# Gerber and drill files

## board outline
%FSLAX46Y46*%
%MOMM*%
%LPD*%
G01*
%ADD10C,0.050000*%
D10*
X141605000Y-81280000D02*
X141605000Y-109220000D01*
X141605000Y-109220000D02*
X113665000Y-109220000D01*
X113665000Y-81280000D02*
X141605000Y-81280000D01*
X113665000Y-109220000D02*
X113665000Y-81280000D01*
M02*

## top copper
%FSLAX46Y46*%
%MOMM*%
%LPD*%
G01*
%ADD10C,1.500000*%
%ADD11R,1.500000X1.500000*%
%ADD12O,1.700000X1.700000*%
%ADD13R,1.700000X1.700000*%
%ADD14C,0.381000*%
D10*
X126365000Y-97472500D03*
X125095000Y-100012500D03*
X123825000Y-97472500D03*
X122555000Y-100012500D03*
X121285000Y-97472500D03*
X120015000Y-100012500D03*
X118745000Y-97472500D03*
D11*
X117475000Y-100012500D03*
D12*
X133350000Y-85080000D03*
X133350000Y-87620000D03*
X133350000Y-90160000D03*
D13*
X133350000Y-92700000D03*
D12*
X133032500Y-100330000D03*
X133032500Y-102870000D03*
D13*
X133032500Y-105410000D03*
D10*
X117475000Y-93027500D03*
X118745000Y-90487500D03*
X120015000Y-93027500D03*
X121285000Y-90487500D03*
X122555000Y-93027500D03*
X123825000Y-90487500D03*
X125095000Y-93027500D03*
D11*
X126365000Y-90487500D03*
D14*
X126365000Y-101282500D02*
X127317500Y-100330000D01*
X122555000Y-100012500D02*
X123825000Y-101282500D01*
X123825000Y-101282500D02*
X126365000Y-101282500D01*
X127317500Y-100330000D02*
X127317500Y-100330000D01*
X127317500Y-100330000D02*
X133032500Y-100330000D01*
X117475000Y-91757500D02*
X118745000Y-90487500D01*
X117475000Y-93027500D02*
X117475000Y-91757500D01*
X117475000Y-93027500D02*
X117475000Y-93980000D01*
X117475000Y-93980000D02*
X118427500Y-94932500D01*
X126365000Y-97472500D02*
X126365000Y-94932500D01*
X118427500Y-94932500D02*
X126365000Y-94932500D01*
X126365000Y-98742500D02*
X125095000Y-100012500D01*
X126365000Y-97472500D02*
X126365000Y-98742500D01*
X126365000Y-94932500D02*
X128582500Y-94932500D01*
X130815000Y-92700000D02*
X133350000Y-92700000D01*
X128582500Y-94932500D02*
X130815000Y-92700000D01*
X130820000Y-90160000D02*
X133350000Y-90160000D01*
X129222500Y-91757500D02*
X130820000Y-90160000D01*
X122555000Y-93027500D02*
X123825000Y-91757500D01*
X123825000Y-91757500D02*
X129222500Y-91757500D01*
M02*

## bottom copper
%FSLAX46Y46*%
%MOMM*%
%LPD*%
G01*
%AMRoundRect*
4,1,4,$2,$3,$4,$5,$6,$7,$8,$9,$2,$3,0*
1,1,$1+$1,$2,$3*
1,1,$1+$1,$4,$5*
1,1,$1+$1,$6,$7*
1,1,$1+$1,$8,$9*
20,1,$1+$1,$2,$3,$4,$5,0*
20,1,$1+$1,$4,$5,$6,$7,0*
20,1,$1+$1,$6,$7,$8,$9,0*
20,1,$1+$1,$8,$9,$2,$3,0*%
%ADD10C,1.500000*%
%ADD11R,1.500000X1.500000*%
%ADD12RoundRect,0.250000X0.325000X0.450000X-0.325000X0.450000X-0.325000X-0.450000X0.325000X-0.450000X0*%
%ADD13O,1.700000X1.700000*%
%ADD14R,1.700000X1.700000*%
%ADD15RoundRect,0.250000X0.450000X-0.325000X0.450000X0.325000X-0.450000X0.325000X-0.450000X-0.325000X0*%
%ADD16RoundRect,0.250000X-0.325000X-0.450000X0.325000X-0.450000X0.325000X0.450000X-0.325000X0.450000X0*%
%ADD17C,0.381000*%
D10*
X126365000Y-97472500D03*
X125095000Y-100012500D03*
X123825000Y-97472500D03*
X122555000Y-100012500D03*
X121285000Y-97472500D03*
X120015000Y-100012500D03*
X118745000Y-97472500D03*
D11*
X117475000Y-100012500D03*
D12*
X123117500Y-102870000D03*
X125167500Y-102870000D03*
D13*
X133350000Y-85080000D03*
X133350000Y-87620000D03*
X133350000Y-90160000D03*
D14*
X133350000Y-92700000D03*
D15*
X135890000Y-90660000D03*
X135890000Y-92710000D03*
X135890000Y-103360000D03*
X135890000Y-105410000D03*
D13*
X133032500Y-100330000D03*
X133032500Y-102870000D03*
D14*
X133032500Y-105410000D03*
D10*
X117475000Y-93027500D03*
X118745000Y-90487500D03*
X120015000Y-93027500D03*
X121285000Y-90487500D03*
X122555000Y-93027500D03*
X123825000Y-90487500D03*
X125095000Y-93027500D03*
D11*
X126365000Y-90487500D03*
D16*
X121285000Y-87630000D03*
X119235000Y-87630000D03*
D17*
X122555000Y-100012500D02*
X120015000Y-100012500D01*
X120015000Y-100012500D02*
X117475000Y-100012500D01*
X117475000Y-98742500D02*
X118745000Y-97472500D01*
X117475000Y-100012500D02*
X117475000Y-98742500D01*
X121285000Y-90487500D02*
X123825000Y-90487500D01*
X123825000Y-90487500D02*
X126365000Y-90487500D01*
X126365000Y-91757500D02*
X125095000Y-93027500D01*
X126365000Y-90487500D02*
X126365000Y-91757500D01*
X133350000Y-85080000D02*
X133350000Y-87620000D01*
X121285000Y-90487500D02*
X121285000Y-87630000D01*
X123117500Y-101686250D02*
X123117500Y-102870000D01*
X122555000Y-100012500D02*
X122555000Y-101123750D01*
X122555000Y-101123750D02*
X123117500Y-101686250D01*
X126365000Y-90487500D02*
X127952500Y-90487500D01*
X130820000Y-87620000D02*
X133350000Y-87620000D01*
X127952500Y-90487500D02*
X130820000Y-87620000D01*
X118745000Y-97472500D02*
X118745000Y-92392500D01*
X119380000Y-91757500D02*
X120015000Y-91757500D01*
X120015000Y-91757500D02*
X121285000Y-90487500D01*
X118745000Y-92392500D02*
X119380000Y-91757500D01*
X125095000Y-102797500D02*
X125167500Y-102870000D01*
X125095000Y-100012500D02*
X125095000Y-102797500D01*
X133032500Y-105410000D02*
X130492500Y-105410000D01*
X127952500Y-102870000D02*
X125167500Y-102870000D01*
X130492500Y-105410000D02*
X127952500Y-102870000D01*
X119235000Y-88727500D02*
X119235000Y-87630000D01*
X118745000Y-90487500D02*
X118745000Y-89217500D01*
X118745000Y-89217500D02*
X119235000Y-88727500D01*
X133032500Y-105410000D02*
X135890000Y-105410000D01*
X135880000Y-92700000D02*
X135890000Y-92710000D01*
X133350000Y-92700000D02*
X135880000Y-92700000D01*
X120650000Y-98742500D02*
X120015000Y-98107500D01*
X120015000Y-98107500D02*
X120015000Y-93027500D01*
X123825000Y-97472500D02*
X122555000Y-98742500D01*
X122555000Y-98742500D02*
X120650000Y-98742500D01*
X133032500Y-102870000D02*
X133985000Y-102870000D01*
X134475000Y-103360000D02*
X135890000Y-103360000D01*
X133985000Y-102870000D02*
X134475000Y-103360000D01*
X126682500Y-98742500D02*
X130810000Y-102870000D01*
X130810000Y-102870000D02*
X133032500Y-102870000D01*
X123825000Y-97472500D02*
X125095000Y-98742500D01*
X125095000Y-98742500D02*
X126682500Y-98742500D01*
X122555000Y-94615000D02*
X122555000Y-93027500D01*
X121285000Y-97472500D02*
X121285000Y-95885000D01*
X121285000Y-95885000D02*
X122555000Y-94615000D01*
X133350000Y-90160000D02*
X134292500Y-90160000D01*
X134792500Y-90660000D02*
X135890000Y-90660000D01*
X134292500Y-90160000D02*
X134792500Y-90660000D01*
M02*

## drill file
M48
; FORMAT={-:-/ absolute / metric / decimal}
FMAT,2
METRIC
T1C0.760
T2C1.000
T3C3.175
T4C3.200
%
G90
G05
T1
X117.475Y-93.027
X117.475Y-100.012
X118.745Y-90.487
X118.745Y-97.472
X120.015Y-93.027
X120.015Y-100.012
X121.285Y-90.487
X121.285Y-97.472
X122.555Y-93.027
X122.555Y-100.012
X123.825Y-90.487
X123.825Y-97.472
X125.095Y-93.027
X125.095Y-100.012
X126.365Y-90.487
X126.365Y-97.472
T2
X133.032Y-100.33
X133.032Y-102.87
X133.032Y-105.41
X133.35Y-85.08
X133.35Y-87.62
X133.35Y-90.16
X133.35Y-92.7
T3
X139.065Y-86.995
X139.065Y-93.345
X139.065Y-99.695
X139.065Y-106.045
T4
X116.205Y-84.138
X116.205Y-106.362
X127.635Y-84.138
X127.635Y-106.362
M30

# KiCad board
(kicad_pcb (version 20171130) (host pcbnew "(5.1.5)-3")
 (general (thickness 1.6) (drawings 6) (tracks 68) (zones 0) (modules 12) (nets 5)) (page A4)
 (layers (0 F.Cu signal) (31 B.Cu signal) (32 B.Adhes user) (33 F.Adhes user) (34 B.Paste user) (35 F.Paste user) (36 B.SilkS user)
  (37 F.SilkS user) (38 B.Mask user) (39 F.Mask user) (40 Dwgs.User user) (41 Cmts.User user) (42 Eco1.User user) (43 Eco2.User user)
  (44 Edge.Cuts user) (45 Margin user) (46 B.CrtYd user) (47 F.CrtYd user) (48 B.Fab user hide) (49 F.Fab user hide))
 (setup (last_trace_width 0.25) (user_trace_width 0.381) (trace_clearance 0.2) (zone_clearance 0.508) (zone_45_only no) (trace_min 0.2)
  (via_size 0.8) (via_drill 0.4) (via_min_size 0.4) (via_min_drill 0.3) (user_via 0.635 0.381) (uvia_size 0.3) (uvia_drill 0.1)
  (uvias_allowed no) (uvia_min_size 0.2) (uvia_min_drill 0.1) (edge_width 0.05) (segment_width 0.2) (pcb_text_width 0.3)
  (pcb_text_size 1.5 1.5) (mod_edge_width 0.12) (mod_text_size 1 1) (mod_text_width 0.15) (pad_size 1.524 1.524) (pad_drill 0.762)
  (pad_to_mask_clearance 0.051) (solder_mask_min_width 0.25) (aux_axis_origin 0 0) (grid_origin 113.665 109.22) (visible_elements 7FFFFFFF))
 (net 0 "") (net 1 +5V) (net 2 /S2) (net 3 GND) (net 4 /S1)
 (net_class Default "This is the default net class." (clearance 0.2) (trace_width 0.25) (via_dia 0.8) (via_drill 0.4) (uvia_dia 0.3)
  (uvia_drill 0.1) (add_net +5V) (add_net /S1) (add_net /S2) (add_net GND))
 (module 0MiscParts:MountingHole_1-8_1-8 (layer F.Cu) (at 139.065 106.045)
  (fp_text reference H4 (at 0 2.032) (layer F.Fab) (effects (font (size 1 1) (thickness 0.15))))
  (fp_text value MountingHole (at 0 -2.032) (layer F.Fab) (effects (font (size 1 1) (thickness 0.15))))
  (pad "" np_thru_hole circle (at 0 0) (size 3.175 3.175) (drill 3.175) (layers *.Cu *.Mask)))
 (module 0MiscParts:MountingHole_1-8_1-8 (layer F.Cu) (at 139.065 86.995)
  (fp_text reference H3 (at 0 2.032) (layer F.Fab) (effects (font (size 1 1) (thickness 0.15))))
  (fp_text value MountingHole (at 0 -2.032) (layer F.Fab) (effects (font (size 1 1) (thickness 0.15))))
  (pad "" np_thru_hole circle (at 0 0) (size 3.175 3.175) (drill 3.175) (layers *.Cu *.Mask)))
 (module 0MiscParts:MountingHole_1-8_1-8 (layer F.Cu) (at 139.065 99.695)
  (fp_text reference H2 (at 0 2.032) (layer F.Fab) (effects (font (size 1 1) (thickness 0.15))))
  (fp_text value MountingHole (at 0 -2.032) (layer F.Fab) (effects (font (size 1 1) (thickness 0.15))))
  (pad "" np_thru_hole circle (at 0 0) (size 3.175 3.175) (drill 3.175) (layers *.Cu *.Mask)))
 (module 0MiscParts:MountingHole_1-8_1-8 (layer F.Cu) (at 139.065 93.345)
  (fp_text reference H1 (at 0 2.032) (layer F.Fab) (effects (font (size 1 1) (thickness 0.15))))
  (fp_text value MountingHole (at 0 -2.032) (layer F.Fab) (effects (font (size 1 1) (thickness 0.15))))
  (pad "" np_thru_hole circle (at 0 0) (size 3.175 3.175) (drill 3.175) (layers *.Cu *.Mask)))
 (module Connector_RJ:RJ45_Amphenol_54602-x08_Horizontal (layer F.Cu) (at 117.475 100.0125)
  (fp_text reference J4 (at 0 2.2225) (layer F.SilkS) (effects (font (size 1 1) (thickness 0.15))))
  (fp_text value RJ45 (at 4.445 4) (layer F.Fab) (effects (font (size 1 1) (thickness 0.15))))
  (pad 8 thru_hole circle (at 8.89 -2.54) (size 1.5 1.5) (drill 0.76) (layers *.Cu *.Mask) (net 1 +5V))
  (pad 7 thru_hole circle (at 7.62 0) (size 1.5 1.5) (drill 0.76) (layers *.Cu *.Mask) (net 1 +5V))
  (pad 6 thru_hole circle (at 6.35 -2.54) (size 1.5 1.5) (drill 0.76) (layers *.Cu *.Mask) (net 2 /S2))
  (pad 5 thru_hole circle (at 5.08 0) (size 1.5 1.5) (drill 0.76) (layers *.Cu *.Mask) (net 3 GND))
  (pad 4 thru_hole circle (at 3.81 -2.54) (size 1.5 1.5) (drill 0.76) (layers *.Cu *.Mask) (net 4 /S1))
  (pad 3 thru_hole circle (at 2.54 0) (size 1.5 1.5) (drill 0.76) (layers *.Cu *.Mask) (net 3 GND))
  (pad 2 thru_hole circle (at 1.27 -2.54) (size 1.5 1.5) (drill 0.76) (layers *.Cu *.Mask) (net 3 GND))
  (pad 1 thru_hole rect (at 0 0) (size 1.5 1.5) (drill 0.76) (layers *.Cu *.Mask) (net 3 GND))
  (pad "" np_thru_hole circle (at -1.27 6.35) (size 3.2 3.2) (drill 3.2) (layers *.Cu *.Mask))
  (pad "" np_thru_hole circle (at 10.16 6.35) (size 3.2 3.2) (drill 3.2) (layers *.Cu *.Mask)))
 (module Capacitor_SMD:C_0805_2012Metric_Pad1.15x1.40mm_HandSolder (layer B.Cu) (at 124.1425 102.87 180)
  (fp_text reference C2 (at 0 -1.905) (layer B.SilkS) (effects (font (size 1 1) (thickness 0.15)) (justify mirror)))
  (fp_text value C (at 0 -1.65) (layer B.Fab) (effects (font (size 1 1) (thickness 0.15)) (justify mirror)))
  (pad 2 smd roundrect (at 1.025 0 180) (size 1.15 1.4) (layers B.Cu B.Paste B.Mask) (roundrect_rratio 0.217391) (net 3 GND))
  (pad 1 smd roundrect (at -1.025 0 180) (size 1.15 1.4) (layers B.Cu B.Paste B.Mask) (roundrect_rratio 0.217391) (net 1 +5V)))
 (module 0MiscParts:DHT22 (layer F.Cu) (at 133.35 88.9 180)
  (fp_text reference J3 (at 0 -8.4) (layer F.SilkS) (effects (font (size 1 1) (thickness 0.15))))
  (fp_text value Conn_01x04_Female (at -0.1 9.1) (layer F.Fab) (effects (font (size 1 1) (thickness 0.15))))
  (pad 4 thru_hole oval (at 0 3.82 180) (size 1.7 1.7) (drill 1) (layers *.Cu *.Mask) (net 3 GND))
  (pad 3 thru_hole oval (at 0 1.28 180) (size 1.7 1.7) (drill 1) (layers *.Cu *.Mask) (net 3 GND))
  (pad 2 thru_hole oval (at 0 -1.26 180) (size 1.7 1.7) (drill 1) (layers *.Cu *.Mask) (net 4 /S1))
  (pad 1 thru_hole rect (at 0 -3.8 180) (size 1.7 1.7) (drill 1) (layers *.Cu *.Mask) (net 1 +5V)))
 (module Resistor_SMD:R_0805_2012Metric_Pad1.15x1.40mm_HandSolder (layer B.Cu) (at 135.89 91.685 90)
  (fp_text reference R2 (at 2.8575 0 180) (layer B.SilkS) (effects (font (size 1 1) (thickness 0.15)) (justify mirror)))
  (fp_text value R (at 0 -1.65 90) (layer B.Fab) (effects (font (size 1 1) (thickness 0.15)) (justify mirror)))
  (pad 2 smd roundrect (at 1.025 0 90) (size 1.15 1.4) (layers B.Cu B.Paste B.Mask) (roundrect_rratio 0.217391) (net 4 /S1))
  (pad 1 smd roundrect (at -1.025 0 90) (size 1.15 1.4) (layers B.Cu B.Paste B.Mask) (roundrect_rratio 0.217391) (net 1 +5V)))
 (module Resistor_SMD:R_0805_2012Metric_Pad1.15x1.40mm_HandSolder (layer B.Cu) (at 135.89 104.385 90)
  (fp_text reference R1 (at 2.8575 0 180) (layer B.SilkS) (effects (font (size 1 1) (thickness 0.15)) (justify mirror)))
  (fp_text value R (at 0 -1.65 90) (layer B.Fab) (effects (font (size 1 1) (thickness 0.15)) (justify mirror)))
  (pad 2 smd roundrect (at 1.025 0 90) (size 1.15 1.4) (layers B.Cu B.Paste B.Mask) (roundrect_rratio 0.217391) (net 2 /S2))
  (pad 1 smd roundrect (at -1.025 0 90) (size 1.15 1.4) (layers B.Cu B.Paste B.Mask) (roundrect_rratio 0.217391) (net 1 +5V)))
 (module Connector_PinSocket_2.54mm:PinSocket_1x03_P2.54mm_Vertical (layer F.Cu) (at 133.0325 105.41 180)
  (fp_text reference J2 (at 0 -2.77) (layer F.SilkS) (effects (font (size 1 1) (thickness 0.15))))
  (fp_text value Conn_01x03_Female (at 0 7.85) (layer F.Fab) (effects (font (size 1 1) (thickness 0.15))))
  (pad 3 thru_hole oval (at 0 5.08 180) (size 1.7 1.7) (drill 1) (layers *.Cu *.Mask) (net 3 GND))
  (pad 2 thru_hole oval (at 0 2.54 180) (size 1.7 1.7) (drill 1) (layers *.Cu *.Mask) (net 2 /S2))
  (pad 1 thru_hole rect (at 0 0 180) (size 1.7 1.7) (drill 1) (layers *.Cu *.Mask) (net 1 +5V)))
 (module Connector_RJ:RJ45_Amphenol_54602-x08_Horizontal (layer F.Cu) (at 126.365 90.4875 180)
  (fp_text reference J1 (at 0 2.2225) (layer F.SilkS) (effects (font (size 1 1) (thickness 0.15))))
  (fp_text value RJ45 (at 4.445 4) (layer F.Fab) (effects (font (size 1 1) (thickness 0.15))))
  (pad 8 thru_hole circle (at 8.89 -2.54 180) (size 1.5 1.5) (drill 0.76) (layers *.Cu *.Mask) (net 1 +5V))
  (pad 7 thru_hole circle (at 7.62 0 180) (size 1.5 1.5) (drill 0.76) (layers *.Cu *.Mask) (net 1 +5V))
  (pad 6 thru_hole circle (at 6.35 -2.54 180) (size 1.5 1.5) (drill 0.76) (layers *.Cu *.Mask) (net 2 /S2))
  (pad 5 thru_hole circle (at 5.08 0 180) (size 1.5 1.5) (drill 0.76) (layers *.Cu *.Mask) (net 3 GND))
  (pad 4 thru_hole circle (at 3.81 -2.54 180) (size 1.5 1.5) (drill 0.76) (layers *.Cu *.Mask) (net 4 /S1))
  (pad 3 thru_hole circle (at 2.54 0 180) (size 1.5 1.5) (drill 0.76) (layers *.Cu *.Mask) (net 3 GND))
  (pad 2 thru_hole circle (at 1.27 -2.54 180) (size 1.5 1.5) (drill 0.76) (layers *.Cu *.Mask) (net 3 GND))
  (pad 1 thru_hole rect (at 0 0 180) (size 1.5 1.5) (drill 0.76) (layers *.Cu *.Mask) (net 3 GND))
  (pad "" np_thru_hole circle (at -1.27 6.35 180) (size 3.2 3.2) (drill 3.2) (layers *.Cu *.Mask))
  (pad "" np_thru_hole circle (at 10.16 6.35 180) (size 3.2 3.2) (drill 3.2) (layers *.Cu *.Mask)))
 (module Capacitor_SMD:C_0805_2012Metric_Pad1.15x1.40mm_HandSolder (layer B.Cu) (at 120.26 87.63)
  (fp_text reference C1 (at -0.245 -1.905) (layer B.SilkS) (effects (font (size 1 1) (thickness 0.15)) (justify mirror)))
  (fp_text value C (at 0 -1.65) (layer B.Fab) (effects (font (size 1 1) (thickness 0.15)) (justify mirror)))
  (pad 2 smd roundrect (at 1.025 0) (size 1.15 1.4) (layers B.Cu B.Paste B.Mask) (roundrect_rratio 0.217391) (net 3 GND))
  (pad 1 smd roundrect (at -1.025 0) (size 1.15 1.4) (layers B.Cu B.Paste B.Mask) (roundrect_rratio 0.217391) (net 1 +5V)))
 (gr_line (start 141.605 81.28) (end 141.605 109.22) (layer Edge.Cuts) (width 0.05))
 (gr_line (start 141.605 109.22) (end 113.665 109.22) (layer Edge.Cuts) (width 0.05))
 (gr_line (start 113.665 81.28) (end 141.605 81.28) (layer Edge.Cuts) (width 0.05))
 (gr_line (start 113.665 109.22) (end 113.665 81.28) (layer Edge.Cuts) (width 0.05))
 (segment (start 122.555 100.0125) (end 120.015 100.0125) (width 0.381) (layer B.Cu) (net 3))
 (segment (start 120.015 100.0125) (end 117.475 100.0125) (width 0.381) (layer B.Cu) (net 3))
 (segment (start 117.475 98.7425) (end 118.745 97.4725) (width 0.381) (layer B.Cu) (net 3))
 (segment (start 117.475 100.0125) (end 117.475 98.7425) (width 0.381) (layer B.Cu) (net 3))
 (segment (start 121.285 90.4875) (end 123.825 90.4875) (width 0.381) (layer B.Cu) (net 3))
 (segment (start 123.825 90.4875) (end 126.365 90.4875) (width 0.381) (layer B.Cu) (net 3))
 (segment (start 126.365 91.7575) (end 125.095 93.0275) (width 0.381) (layer B.Cu) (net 3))
 (segment (start 126.365 90.4875) (end 126.365 91.7575) (width 0.381) (layer B.Cu) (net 3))
 (segment (start 133.35 85.08) (end 133.35 87.62) (width 0.381) (layer B.Cu) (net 3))
 (segment (start 121.285 90.4875) (end 121.285 87.63) (width 0.381) (layer B.Cu) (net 3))
 (segment (start 126.365 101.2825) (end 127.3175 100.33) (width 0.381) (layer F.Cu) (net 3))
 (segment (start 122.555 100.0125) (end 123.825 101.2825) (width 0.381) (layer F.Cu) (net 3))
 (segment (start 123.825 101.2825) (end 126.365 101.2825) (width 0.381) (layer F.Cu) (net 3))
 (segment (start 127.3175 100.33) (end 127.3175 100.33) (width 0.381) (layer F.Cu) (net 3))
 (segment (start 123.1175 101.68625) (end 123.1175 102.87) (width 0.381) (layer B.Cu) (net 3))
 (segment (start 122.555 100.0125) (end 122.555 101.12375) (width 0.381) (layer B.Cu) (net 3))
 (segment (start 122.555 101.12375) (end 123.1175 101.68625) (width 0.381) (layer B.Cu) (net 3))
 (segment (start 126.365 90.4875) (end 127.9525 90.4875) (width 0.381) (layer B.Cu) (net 3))
 (segment (start 130.82 87.62) (end 133.35 87.62) (width 0.381) (layer B.Cu) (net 3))
 (segment (start 127.9525 90.4875) (end 130.82 87.62) (width 0.381) (layer B.Cu) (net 3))
 (segment (start 118.745 97.4725) (end 118.745 92.3925) (width 0.381) (layer B.Cu) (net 3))
 (segment (start 119.38 91.7575) (end 120.015 91.7575) (width 0.381) (layer B.Cu) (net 3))
 (segment (start 120.015 91.7575) (end 121.285 90.4875) (width 0.381) (layer B.Cu) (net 3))
 (segment (start 118.745 92.3925) (end 119.38 91.7575) (width 0.381) (layer B.Cu) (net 3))
 (segment (start 127.3175 100.33) (end 133.0325 100.33) (width 0.381) (layer F.Cu) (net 3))
 (segment (start 125.095 102.7975) (end 125.1675 102.87) (width 0.381) (layer B.Cu) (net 1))
 (segment (start 125.095 100.0125) (end 125.095 102.7975) (width 0.381) (layer B.Cu) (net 1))
 (segment (start 133.0325 105.41) (end 130.4925 105.41) (width 0.381) (layer B.Cu) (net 1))
 (segment (start 127.9525 102.87) (end 125.1675 102.87) (width 0.381) (layer B.Cu) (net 1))
 (segment (start 130.4925 105.41) (end 127.9525 102.87) (width 0.381) (layer B.Cu) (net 1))
 (segment (start 119.235 88.7275) (end 119.235 87.63) (width 0.381) (layer B.Cu) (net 1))
 (segment (start 118.745 90.4875) (end 118.745 89.2175) (width 0.381) (layer B.Cu) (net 1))
 (segment (start 118.745 89.2175) (end 119.235 88.7275) (width 0.381) (layer B.Cu) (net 1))
 (segment (start 117.475 91.7575) (end 118.745 90.4875) (width 0.381) (layer F.Cu) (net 1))
 (segment (start 117.475 93.0275) (end 117.475 91.7575) (width 0.381) (layer F.Cu) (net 1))
 (segment (start 117.475 93.0275) (end 117.475 93.98) (width 0.381) (layer F.Cu) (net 1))
 (segment (start 117.475 93.98) (end 118.4275 94.9325) (width 0.381) (layer F.Cu) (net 1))
 (segment (start 126.365 97.4725) (end 126.365 94.9325) (width 0.381) (layer F.Cu) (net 1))
 (segment (start 118.4275 94.9325) (end 126.365 94.9325) (width 0.381) (layer F.Cu) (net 1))
 (segment (start 126.365 98.7425) (end 125.095 100.0125) (width 0.381) (layer F.Cu) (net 1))
 (segment (start 126.365 97.4725) (end 126.365 98.7425) (width 0.381) (layer F.Cu) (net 1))
 (segment (start 133.0325 105.41) (end 135.89 105.41) (width 0.381) (layer B.Cu) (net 1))
 (segment (start 135.88 92.7) (end 135.89 92.71) (width 0.381) (layer B.Cu) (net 1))
 (segment (start 133.35 92.7) (end 135.88 92.7) (width 0.381) (layer B.Cu) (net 1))
 (segment (start 126.365 94.9325) (end 128.5825 94.9325) (width 0.381) (layer F.Cu) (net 1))
 (segment (start 130.815 92.7) (end 133.35 92.7) (width 0.381) (layer F.Cu) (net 1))
 (segment (start 128.5825 94.9325) (end 130.815 92.7) (width 0.381) (layer F.Cu) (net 1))
 (segment (start 120.65 98.7425) (end 120.015 98.1075) (width 0.381) (layer B.Cu) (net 2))
 (segment (start 120.015 98.1075) (end 120.015 93.0275) (width 0.381) (layer B.Cu) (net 2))
 (segment (start 123.825 97.4725) (end 122.555 98.7425) (width 0.381) (layer B.Cu) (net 2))
 (segment (start 122.555 98.7425) (end 120.65 98.7425) (width 0.381) (layer B.Cu) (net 2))
 (segment (start 133.0325 102.87) (end 133.985 102.87) (width 0.381) (layer B.Cu) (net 2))
 (segment (start 134.475 103.36) (end 135.89 103.36) (width 0.381) (layer B.Cu) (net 2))
 (segment (start 133.985 102.87) (end 134.475 103.36) (width 0.381) (layer B.Cu) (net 2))
 (segment (start 126.6825 98.7425) (end 130.81 102.87) (width 0.381) (layer B.Cu) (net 2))
 (segment (start 130.81 102.87) (end 133.0325 102.87) (width 0.381) (layer B.Cu) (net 2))
 (segment (start 123.825 97.4725) (end 125.095 98.7425) (width 0.381) (layer B.Cu) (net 2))
 (segment (start 125.095 98.7425) (end 126.6825 98.7425) (width 0.381) (layer B.Cu) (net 2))
 (segment (start 130.82 90.16) (end 133.35 90.16) (width 0.381) (layer F.Cu) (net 4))
 (segment (start 129.2225 91.7575) (end 130.82 90.16) (width 0.381) (layer F.Cu) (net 4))
 (segment (start 122.555 93.0275) (end 123.825 91.7575) (width 0.381) (layer F.Cu) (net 4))
 (segment (start 123.825 91.7575) (end 129.2225 91.7575) (width 0.381) (layer F.Cu) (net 4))
 (segment (start 122.555 94.615) (end 122.555 93.0275) (width 0.381) (layer B.Cu) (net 4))
 (segment (start 121.285 97.4725) (end 121.285 95.885) (width 0.381) (layer B.Cu) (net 4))
 (segment (start 121.285 95.885) (end 122.555 94.615) (width 0.381) (layer B.Cu) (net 4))
 (segment (start 133.35 90.16) (end 134.2925 90.16) (width 0.381) (layer B.Cu) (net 4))
 (segment (start 134.7925 90.66) (end 135.89 90.66) (width 0.381) (layer B.Cu) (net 4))
 (segment (start 134.2925 90.16) (end 134.7925 90.66) (width 0.381) (layer B.Cu) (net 4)))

